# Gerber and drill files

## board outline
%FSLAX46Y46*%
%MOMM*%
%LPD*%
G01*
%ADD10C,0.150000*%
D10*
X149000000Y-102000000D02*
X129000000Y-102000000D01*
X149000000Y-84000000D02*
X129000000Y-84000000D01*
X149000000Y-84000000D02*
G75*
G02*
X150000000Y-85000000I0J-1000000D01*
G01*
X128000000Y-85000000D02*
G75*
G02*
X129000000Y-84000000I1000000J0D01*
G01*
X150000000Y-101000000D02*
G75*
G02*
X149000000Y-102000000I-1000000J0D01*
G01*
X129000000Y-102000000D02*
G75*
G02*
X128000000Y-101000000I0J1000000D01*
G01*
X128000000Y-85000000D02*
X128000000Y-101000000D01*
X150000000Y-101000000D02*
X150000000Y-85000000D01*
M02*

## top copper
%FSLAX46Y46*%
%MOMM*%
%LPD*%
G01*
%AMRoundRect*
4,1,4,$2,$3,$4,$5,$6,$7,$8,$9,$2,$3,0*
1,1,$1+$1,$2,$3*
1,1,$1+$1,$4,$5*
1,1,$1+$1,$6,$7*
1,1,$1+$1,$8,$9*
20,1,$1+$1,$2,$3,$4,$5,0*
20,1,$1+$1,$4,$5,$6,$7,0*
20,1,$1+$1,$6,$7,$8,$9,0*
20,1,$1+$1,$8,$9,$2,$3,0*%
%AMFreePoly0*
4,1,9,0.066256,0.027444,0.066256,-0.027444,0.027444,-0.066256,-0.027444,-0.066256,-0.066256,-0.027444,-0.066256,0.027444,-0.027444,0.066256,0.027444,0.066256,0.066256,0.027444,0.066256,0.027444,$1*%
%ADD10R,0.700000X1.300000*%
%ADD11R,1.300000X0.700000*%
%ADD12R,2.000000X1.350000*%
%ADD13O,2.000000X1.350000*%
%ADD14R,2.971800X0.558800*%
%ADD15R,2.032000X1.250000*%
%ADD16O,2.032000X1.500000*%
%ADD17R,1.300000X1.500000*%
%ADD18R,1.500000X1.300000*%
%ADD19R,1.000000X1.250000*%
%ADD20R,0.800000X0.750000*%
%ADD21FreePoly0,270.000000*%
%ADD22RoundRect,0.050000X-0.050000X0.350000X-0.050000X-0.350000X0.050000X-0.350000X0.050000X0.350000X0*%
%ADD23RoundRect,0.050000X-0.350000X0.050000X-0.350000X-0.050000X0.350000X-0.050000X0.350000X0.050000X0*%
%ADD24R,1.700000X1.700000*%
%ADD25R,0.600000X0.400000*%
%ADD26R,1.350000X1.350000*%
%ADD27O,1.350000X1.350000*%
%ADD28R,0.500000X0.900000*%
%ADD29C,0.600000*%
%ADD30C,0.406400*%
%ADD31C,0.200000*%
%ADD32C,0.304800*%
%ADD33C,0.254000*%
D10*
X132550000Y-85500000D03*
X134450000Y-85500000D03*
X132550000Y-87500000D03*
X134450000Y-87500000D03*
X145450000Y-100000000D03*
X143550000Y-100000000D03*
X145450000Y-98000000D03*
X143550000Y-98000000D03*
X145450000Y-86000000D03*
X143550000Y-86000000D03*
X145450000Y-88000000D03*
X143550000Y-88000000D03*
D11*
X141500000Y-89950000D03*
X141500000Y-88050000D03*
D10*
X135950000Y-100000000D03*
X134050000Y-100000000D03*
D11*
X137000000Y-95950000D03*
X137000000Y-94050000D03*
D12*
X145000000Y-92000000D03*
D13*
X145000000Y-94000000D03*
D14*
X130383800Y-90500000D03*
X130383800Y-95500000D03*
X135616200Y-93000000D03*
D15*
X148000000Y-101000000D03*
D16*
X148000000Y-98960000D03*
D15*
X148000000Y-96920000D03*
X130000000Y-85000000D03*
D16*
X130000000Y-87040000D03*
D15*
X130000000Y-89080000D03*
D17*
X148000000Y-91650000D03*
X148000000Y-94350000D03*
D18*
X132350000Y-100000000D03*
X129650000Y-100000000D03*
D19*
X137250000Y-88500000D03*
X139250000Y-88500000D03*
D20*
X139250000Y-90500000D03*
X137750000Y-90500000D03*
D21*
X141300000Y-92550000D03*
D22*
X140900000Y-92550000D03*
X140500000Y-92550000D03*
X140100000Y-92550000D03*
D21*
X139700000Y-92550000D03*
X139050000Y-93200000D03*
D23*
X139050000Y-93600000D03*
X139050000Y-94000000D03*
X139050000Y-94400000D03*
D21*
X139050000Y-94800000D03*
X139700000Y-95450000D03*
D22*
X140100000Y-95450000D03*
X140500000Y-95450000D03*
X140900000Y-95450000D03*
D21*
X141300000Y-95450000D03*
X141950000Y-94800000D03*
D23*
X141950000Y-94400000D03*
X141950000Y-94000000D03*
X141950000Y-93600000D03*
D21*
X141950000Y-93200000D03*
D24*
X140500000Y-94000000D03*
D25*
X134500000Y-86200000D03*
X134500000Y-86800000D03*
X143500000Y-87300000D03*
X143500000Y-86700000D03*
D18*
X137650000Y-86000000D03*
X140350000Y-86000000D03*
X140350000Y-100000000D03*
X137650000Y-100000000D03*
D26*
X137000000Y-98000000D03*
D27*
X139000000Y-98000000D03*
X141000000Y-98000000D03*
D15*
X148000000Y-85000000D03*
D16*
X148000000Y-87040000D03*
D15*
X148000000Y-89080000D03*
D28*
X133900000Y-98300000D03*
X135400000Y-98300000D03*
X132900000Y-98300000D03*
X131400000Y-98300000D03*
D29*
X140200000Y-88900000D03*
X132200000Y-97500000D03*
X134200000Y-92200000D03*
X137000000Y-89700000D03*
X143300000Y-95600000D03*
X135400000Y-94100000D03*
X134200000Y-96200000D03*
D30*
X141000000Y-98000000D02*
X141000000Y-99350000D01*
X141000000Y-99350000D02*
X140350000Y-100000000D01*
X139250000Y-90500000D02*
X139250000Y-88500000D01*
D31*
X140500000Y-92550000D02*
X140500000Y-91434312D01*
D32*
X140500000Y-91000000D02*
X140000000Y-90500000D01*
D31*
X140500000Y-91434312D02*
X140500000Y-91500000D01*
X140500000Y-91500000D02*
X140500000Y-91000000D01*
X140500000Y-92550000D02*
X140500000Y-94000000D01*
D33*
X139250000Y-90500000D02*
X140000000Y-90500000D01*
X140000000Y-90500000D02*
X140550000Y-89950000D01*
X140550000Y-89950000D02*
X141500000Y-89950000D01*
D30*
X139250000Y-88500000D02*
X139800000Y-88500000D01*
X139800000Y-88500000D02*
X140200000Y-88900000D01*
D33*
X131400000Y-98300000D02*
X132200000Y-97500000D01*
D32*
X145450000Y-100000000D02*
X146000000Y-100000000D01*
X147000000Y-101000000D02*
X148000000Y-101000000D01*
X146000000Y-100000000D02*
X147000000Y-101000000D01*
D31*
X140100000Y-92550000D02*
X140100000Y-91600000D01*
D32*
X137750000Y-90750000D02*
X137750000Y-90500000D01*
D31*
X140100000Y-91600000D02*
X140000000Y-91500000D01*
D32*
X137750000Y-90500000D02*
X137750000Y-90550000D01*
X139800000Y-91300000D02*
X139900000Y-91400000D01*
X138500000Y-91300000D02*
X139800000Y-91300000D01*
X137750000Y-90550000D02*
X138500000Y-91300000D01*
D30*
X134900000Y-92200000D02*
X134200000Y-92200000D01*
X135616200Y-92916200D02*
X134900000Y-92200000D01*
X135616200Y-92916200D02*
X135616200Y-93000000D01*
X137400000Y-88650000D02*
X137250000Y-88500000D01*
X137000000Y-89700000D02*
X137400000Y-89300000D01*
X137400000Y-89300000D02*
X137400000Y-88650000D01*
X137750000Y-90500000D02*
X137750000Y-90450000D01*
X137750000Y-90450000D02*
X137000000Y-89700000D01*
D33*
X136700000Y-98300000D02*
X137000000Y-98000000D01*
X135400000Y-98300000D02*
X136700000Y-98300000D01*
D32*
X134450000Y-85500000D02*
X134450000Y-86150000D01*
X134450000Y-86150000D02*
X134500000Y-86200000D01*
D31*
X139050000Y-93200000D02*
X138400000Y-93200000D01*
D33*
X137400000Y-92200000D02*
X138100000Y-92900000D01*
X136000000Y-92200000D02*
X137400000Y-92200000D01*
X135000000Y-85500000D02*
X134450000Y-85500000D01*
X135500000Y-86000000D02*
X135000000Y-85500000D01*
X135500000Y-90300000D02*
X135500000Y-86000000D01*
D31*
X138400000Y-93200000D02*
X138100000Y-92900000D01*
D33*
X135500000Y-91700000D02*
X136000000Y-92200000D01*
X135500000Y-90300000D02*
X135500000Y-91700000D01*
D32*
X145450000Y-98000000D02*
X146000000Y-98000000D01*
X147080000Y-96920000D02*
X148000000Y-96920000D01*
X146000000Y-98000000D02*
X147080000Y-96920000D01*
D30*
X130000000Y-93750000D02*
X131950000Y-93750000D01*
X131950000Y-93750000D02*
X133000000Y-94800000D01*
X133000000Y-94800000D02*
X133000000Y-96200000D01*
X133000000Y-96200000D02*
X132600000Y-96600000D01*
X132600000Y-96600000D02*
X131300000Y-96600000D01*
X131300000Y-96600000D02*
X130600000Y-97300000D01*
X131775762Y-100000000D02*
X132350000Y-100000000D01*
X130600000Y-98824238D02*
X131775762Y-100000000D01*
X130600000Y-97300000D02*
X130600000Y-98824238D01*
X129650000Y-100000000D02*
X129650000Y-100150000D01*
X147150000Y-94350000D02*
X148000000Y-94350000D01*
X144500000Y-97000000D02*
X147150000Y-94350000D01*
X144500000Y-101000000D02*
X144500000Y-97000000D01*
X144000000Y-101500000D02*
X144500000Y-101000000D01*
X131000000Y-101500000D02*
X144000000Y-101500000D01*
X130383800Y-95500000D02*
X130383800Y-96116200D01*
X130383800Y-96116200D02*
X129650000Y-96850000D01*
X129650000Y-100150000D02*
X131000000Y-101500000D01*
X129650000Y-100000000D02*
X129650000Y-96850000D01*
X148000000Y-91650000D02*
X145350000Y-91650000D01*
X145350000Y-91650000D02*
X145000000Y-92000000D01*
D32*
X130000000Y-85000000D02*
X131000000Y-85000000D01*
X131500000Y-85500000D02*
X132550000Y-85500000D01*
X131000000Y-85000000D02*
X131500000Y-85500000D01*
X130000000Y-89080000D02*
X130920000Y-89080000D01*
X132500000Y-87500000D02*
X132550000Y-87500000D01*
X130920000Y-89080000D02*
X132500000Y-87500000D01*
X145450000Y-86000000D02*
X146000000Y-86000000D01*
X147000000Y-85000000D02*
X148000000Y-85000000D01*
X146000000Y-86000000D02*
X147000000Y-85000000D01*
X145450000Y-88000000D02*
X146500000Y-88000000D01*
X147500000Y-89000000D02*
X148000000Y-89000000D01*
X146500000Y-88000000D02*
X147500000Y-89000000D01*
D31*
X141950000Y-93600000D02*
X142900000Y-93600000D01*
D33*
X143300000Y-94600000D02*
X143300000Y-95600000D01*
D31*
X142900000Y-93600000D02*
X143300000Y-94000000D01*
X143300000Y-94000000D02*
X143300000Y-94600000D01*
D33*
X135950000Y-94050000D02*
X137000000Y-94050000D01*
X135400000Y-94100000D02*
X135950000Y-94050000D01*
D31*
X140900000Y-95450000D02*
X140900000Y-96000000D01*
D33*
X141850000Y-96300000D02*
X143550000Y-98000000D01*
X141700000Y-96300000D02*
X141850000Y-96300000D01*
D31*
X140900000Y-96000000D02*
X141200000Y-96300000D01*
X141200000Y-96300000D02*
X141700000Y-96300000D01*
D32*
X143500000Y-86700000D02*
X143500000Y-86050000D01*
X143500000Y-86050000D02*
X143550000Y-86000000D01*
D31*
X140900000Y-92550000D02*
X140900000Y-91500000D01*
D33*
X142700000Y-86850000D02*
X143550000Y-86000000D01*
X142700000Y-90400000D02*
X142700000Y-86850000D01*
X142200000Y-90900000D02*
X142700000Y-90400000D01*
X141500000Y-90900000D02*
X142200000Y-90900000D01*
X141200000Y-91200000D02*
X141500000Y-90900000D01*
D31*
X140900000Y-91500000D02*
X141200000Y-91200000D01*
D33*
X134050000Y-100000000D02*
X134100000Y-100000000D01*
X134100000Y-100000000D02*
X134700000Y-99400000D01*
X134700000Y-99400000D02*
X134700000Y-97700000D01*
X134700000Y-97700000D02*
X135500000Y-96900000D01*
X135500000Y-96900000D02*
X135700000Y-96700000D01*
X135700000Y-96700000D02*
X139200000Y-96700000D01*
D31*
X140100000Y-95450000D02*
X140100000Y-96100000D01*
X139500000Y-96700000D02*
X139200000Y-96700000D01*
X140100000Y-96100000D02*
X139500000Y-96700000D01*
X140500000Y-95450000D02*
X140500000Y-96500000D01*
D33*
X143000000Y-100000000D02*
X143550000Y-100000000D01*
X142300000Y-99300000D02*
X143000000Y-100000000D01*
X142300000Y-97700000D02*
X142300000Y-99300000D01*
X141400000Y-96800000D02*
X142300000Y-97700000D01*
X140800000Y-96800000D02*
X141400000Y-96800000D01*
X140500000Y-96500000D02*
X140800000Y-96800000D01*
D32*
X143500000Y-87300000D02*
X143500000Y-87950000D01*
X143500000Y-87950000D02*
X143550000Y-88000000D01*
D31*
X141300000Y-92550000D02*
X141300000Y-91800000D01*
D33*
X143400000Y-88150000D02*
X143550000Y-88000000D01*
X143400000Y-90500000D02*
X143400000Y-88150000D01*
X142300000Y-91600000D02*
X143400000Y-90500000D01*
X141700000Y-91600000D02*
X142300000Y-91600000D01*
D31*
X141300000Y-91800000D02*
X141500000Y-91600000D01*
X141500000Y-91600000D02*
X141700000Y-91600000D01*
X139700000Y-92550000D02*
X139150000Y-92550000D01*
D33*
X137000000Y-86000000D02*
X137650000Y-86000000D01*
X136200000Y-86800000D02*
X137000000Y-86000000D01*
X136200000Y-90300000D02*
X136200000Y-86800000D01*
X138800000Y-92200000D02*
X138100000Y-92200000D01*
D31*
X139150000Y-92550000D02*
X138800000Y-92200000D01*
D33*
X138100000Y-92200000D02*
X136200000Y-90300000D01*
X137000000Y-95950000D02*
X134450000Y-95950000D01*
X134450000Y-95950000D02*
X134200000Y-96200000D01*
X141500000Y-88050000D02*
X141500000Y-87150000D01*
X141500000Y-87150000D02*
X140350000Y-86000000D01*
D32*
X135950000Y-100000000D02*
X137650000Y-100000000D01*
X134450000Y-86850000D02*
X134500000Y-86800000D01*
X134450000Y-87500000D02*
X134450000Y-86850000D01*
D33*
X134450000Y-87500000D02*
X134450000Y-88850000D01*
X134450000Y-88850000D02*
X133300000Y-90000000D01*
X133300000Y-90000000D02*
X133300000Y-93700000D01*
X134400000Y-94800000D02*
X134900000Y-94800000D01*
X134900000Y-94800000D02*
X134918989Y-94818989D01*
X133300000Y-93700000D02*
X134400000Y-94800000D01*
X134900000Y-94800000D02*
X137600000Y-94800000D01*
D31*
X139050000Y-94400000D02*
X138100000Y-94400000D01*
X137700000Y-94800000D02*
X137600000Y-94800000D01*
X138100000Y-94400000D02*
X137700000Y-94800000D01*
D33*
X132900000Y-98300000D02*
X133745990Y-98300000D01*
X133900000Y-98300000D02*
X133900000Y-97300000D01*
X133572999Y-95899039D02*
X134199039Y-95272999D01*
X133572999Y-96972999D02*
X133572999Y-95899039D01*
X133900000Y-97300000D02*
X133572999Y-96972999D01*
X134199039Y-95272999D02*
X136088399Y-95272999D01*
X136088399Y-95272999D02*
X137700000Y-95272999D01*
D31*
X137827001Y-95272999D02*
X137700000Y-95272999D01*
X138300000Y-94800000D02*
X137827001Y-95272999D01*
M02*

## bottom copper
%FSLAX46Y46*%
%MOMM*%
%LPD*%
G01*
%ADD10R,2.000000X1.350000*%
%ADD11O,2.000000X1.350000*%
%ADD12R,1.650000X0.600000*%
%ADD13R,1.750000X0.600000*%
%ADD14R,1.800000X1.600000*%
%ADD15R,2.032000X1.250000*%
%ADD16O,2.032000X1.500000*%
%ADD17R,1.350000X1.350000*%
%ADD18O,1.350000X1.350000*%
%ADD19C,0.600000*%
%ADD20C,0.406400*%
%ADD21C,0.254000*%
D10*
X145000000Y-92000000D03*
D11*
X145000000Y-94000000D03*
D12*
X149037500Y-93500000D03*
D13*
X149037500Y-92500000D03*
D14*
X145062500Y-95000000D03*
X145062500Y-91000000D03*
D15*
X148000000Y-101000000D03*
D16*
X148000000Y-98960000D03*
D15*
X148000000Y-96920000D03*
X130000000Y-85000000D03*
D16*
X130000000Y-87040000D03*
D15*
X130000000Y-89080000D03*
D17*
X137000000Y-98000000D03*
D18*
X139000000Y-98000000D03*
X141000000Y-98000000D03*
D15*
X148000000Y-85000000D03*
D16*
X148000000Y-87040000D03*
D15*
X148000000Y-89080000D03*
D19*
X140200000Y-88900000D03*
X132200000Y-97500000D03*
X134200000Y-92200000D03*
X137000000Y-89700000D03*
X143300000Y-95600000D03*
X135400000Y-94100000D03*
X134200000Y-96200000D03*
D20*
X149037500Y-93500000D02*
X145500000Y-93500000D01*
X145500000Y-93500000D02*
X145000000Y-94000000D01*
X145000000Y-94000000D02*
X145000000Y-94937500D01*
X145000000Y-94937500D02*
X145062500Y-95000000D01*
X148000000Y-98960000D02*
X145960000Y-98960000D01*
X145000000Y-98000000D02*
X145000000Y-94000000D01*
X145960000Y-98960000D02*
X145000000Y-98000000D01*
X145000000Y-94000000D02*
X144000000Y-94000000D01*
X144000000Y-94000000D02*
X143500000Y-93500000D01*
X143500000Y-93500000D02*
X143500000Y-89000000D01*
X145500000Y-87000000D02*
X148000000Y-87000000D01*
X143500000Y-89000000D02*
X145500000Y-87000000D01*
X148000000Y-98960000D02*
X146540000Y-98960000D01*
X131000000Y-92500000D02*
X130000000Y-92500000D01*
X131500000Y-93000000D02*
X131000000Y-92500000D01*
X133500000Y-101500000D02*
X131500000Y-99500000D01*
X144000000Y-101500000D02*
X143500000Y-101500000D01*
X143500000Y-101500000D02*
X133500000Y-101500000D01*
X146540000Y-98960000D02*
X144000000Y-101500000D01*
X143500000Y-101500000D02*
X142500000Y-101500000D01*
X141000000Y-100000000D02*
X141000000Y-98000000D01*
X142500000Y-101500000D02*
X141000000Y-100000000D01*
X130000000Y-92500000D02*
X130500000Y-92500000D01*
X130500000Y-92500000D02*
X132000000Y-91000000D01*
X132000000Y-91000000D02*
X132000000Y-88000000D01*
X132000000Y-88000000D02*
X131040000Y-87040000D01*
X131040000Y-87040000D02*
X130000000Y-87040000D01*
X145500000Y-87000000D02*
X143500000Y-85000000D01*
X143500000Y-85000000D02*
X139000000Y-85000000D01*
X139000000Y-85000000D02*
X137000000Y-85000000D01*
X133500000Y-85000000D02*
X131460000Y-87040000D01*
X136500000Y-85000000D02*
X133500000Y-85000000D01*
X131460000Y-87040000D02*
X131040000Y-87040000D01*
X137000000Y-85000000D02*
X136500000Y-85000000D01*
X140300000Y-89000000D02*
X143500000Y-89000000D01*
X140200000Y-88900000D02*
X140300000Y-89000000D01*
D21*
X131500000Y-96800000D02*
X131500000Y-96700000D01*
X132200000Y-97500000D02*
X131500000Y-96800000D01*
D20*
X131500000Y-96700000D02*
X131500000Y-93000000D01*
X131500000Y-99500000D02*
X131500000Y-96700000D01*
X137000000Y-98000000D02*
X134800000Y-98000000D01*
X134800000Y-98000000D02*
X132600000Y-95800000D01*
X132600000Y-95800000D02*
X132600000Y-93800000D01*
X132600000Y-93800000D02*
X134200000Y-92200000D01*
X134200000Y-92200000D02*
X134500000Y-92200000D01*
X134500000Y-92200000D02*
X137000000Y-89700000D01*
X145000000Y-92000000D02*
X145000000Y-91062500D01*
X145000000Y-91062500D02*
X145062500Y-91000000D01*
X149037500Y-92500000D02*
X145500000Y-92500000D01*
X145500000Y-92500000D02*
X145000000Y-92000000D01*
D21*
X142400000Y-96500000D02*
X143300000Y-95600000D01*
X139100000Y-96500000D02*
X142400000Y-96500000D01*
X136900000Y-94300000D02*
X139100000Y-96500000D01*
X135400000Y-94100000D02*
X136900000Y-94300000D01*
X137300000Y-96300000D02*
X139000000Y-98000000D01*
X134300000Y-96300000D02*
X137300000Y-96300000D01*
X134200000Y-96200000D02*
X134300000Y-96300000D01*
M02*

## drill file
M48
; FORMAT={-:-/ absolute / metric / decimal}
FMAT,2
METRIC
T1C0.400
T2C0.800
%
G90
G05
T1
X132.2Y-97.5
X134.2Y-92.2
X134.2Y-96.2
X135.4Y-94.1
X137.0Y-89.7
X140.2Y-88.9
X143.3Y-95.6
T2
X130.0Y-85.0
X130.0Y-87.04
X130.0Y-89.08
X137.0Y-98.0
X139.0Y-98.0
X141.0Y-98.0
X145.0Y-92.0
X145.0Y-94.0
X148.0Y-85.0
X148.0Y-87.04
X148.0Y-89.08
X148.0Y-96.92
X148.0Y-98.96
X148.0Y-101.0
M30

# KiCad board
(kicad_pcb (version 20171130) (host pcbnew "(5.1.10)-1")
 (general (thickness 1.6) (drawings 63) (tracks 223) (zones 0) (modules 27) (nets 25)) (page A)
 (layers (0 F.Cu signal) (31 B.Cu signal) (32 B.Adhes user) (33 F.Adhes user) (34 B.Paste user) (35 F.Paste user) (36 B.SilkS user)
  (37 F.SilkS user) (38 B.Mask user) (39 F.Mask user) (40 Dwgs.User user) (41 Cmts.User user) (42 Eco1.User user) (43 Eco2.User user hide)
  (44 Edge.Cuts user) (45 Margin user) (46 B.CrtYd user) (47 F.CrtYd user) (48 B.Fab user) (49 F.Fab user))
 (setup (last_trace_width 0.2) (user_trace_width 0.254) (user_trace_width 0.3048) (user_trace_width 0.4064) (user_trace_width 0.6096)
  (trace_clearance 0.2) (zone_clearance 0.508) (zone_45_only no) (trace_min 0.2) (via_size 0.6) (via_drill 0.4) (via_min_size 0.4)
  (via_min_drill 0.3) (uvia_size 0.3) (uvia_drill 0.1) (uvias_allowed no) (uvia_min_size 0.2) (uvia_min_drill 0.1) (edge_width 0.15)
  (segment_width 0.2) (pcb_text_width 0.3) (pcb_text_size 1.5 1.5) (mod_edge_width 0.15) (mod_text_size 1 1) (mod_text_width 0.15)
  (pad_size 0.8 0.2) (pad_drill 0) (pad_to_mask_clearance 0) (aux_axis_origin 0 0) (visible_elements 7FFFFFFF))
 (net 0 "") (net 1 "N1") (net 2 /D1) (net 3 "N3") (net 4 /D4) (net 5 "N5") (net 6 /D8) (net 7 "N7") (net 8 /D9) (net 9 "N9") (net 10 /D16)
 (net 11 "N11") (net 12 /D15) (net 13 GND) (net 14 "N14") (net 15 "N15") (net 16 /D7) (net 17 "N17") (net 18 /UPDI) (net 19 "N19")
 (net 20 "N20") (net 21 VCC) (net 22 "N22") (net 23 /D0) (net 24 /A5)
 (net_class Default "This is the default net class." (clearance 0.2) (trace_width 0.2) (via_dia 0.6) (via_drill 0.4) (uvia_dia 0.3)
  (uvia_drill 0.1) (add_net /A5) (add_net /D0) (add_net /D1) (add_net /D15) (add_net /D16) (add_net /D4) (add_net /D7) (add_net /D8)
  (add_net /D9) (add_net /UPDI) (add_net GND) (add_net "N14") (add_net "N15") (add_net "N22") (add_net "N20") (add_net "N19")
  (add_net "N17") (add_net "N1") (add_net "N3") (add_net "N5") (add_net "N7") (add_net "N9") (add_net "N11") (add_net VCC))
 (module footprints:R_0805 (layer F.Cu) (at 133.5 85.5 180)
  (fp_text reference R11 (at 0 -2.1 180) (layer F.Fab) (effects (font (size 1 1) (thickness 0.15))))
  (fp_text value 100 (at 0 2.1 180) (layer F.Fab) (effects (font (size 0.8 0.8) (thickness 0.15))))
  (pad 2 smd rect (at 0.95 0 180) (size 0.7 1.3) (layers F.Cu F.Paste F.Mask) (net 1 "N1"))
  (pad 1 smd rect (at -0.95 0 180) (size 0.7 1.3) (layers F.Cu F.Paste F.Mask) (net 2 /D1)))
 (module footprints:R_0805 (layer F.Cu) (at 133.5 87.5 180)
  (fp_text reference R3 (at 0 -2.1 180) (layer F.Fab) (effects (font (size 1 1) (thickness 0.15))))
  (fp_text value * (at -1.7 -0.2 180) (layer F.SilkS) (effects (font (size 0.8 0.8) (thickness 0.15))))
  (pad 2 smd rect (at 0.95 0 180) (size 0.7 1.3) (layers F.Cu F.Paste F.Mask) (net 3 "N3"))
  (pad 1 smd rect (at -0.95 0 180) (size 0.7 1.3) (layers F.Cu F.Paste F.Mask) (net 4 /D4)))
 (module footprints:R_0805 (layer F.Cu) (at 144.5 100)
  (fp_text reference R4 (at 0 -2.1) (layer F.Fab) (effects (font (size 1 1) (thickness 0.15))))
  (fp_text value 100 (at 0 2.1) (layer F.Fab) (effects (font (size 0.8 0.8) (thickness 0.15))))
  (pad 2 smd rect (at 0.95 0) (size 0.7 1.3) (layers F.Cu F.Paste F.Mask) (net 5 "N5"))
  (pad 1 smd rect (at -0.95 0) (size 0.7 1.3) (layers F.Cu F.Paste F.Mask) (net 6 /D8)))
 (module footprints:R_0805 (layer F.Cu) (at 144.5 98)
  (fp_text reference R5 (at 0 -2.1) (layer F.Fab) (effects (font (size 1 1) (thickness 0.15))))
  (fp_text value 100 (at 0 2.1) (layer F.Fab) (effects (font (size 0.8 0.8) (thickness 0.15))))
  (pad 2 smd rect (at 0.95 0) (size 0.7 1.3) (layers F.Cu F.Paste F.Mask) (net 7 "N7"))
  (pad 1 smd rect (at -0.95 0) (size 0.7 1.3) (layers F.Cu F.Paste F.Mask) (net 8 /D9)))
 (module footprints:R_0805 (layer F.Cu) (at 144.5 86)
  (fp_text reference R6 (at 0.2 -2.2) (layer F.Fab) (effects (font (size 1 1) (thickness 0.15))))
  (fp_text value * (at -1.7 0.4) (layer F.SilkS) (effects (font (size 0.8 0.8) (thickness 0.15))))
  (pad 2 smd rect (at 0.95 0) (size 0.7 1.3) (layers F.Cu F.Paste F.Mask) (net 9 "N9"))
  (pad 1 smd rect (at -0.95 0) (size 0.7 1.3) (layers F.Cu F.Paste F.Mask) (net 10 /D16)))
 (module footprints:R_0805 (layer F.Cu) (at 144.5 88)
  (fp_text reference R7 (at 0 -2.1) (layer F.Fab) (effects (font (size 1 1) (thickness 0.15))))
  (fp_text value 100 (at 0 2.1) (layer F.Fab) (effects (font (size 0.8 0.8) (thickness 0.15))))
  (pad 2 smd rect (at 0.95 0) (size 0.7 1.3) (layers F.Cu F.Paste F.Mask) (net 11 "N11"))
  (pad 1 smd rect (at -0.95 0) (size 0.7 1.3) (layers F.Cu F.Paste F.Mask) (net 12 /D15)))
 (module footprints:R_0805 (layer F.Cu) (at 141.5 89 270)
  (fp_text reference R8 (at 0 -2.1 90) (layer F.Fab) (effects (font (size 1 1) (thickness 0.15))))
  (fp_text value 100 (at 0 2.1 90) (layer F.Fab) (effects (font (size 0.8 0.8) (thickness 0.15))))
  (pad 2 smd rect (at 0.95 0 270) (size 0.7 1.3) (layers F.Cu F.Paste F.Mask) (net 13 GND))
  (pad 1 smd rect (at -0.95 0 270) (size 0.7 1.3) (layers F.Cu F.Paste F.Mask) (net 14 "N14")))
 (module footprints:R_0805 (layer F.Cu) (at 135 100)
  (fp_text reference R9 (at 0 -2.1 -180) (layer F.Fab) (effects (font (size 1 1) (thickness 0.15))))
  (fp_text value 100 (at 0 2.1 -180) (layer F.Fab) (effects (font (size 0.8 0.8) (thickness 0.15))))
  (pad 2 smd rect (at 0.95 0) (size 0.7 1.3) (layers F.Cu F.Paste F.Mask) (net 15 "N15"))
  (pad 1 smd rect (at -0.95 0) (size 0.7 1.3) (layers F.Cu F.Paste F.Mask) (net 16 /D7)))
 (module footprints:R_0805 (layer F.Cu) (at 137 95 270)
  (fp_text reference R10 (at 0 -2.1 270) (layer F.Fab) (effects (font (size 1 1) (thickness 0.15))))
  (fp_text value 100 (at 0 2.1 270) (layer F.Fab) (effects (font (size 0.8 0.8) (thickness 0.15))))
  (pad 2 smd rect (at 0.95 0 270) (size 0.7 1.3) (layers F.Cu F.Paste F.Mask) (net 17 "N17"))
  (pad 1 smd rect (at -0.95 0 270) (size 0.7 1.3) (layers F.Cu F.Paste F.Mask) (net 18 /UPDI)))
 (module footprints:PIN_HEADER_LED (layer B.Cu) (at 145 92 180)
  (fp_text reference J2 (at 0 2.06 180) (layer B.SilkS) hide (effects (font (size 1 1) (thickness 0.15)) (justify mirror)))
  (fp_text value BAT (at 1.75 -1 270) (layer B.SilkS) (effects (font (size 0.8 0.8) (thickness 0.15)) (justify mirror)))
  (pad 1 thru_hole rect (at 0 0 180) (size 2 1.35) (drill 0.8) (layers *.Cu *.Mask) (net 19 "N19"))
  (pad 2 thru_hole oval (at 0 -2 180) (size 2 1.35) (drill 0.8) (layers *.Cu *.Mask) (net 13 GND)))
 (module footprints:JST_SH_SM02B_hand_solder (layer B.Cu) (at 147 93 90)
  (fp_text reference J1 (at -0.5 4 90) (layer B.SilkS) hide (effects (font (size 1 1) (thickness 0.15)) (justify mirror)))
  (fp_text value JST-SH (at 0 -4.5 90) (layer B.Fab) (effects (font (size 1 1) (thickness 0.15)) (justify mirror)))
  (pad 1 smd rect (at -0.5 2.0375 90) (size 0.6 1.65) (layers B.Cu B.Paste B.Mask) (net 13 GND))
  (pad 2 smd rect (at 0.5 2.0375 90) (size 0.6 1.75) (layers B.Cu B.Paste B.Mask) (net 19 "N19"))
  (pad 1 smd rect (at -2 -1.9375 90) (size 1.6 1.8) (layers B.Cu B.Paste B.Mask) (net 13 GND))
  (pad 2 smd rect (at 2 -1.9375 90) (size 1.6 1.8) (layers B.Cu B.Paste B.Mask) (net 19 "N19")))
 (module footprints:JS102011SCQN (layer F.Cu) (at 133 93)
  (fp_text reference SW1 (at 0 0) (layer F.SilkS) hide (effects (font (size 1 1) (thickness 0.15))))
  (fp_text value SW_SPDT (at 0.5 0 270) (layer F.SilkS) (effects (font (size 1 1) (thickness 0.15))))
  (pad 1 smd rect (at -2.6162 -2.5) (size 2.9718 0.5588) (layers F.Cu F.Paste F.Mask))
  (pad 3 smd rect (at -2.6162 2.5) (size 2.9718 0.5588) (layers F.Cu F.Paste F.Mask) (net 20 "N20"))
  (pad 2 smd rect (at 2.6162 0) (size 2.9718 0.5588) (layers F.Cu F.Paste F.Mask) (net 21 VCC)))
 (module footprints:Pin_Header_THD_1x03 (layer F.Cu) (at 148 101 180)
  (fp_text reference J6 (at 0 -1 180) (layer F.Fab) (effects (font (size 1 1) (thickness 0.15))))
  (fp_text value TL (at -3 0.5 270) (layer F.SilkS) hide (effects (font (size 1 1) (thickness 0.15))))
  (pad 1 thru_hole rect (at 0 0 180) (size 2.032 1.25) (drill 0.8) (layers *.Cu *.Mask F.SilkS) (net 5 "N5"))
  (pad 2 thru_hole oval (at 0 2.04 180) (size 2.032 1.5) (drill 0.8) (layers *.Cu *.Mask F.SilkS) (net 13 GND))
  (pad 3 thru_hole rect (at 0 4.08 180) (size 2.032 1.25) (drill 0.8) (layers *.Cu *.Mask F.SilkS) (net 7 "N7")))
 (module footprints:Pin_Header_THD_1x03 (layer F.Cu) (at 130 85)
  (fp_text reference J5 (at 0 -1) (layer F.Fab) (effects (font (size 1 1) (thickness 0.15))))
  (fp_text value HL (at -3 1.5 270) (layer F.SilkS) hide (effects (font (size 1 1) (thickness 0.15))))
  (pad 1 thru_hole rect (at 0 0) (size 2.032 1.25) (drill 0.8) (layers *.Cu *.Mask F.SilkS) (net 1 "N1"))
  (pad 2 thru_hole oval (at 0 2.04) (size 2.032 1.5) (drill 0.8) (layers *.Cu *.Mask F.SilkS) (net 13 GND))
  (pad 3 thru_hole rect (at 0 4.08) (size 2.032 1.25) (drill 0.8) (layers *.Cu *.Mask F.SilkS) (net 3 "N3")))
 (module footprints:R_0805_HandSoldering (layer F.Cu) (at 148 93 270)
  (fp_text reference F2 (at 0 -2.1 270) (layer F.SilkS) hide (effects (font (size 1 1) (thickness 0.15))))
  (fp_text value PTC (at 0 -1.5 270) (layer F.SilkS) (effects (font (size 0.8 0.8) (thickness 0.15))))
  (pad 1 smd rect (at -1.35 0 270) (size 1.5 1.3) (layers F.Cu F.Paste F.Mask) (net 19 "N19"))
  (pad 2 smd rect (at 1.35 0 270) (size 1.5 1.3) (layers F.Cu F.Paste F.Mask) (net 20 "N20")))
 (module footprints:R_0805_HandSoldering (layer F.Cu) (at 131 100 180)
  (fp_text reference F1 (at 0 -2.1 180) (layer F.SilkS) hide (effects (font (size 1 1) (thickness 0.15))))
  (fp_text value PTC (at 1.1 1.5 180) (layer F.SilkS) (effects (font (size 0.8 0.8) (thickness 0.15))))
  (pad 1 smd rect (at -1.35 0 180) (size 1.5 1.3) (layers F.Cu F.Paste F.Mask) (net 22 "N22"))
  (pad 2 smd rect (at 1.35 0 180) (size 1.5 1.3) (layers F.Cu F.Paste F.Mask) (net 20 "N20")))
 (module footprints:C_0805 (layer F.Cu) (at 138.25 88.5)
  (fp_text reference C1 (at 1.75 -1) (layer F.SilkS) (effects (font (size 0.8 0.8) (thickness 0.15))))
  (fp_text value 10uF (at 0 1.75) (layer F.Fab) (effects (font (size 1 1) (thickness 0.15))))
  (pad 1 smd rect (at -1 0) (size 1 1.25) (layers F.Cu F.Paste F.Mask) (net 21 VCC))
  (pad 2 smd rect (at 1 0) (size 1 1.25) (layers F.Cu F.Paste F.Mask) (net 13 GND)))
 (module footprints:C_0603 (layer F.Cu) (at 138.5 90.5)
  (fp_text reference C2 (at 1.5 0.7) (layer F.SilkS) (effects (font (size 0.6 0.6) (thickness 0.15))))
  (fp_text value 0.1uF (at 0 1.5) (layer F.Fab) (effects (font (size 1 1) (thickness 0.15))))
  (pad 2 smd rect (at 0.75 0) (size 0.8 0.75) (layers F.Cu F.Paste F.Mask) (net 13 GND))
  (pad 1 smd rect (at -0.75 0) (size 0.8 0.75) (layers F.Cu F.Paste F.Mask) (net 21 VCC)))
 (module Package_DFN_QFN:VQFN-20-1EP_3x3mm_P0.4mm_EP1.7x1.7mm (layer F.Cu) (at 140.5 94 270)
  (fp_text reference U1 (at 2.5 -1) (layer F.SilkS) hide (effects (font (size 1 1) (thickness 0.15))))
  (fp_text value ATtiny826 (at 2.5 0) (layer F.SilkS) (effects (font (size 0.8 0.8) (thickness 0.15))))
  (pad 1 smd custom (at -1.45 -0.8 270) (size 0.143431 0.143431) (layers F.Cu F.Paste F.Mask) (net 12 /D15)
   (options (clearance outline) (anchor circle)) (primitives))
  (pad 2 smd roundrect (at -1.45 -0.4 270) (size 0.8 0.2) (layers F.Cu F.Paste F.Mask) (roundrect_rratio 0.25) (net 10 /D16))
  (pad 3 smd roundrect (at -1.45 0 270) (size 0.8 0.2) (layers F.Cu F.Paste F.Mask) (roundrect_rratio 0.25) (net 13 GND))
  (pad 4 smd roundrect (at -1.45 0.4 270) (size 0.8 0.2) (layers F.Cu F.Paste F.Mask) (roundrect_rratio 0.25) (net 21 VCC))
  (pad 5 smd custom (at -1.45 0.8 270) (size 0.143431 0.143431) (layers F.Cu F.Paste F.Mask) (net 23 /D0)
   (options (clearance outline) (anchor circle)) (primitives))
  (pad 6 smd custom (at -0.8 1.45 270) (size 0.143431 0.143431) (layers F.Cu F.Paste F.Mask) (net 2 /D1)
   (options (clearance outline) (anchor circle)) (primitives))
  (pad 7 smd roundrect (at -0.4 1.45 270) (size 0.2 0.8) (layers F.Cu F.Paste F.Mask) (roundrect_rratio 0.25))
  (pad 8 smd roundrect (at 0 1.45 270) (size 0.2 0.8) (layers F.Cu F.Paste F.Mask) (roundrect_rratio 0.25))
  (pad 9 smd roundrect (at 0.4 1.45 270) (size 0.2 0.8) (layers F.Cu F.Paste F.Mask) (roundrect_rratio 0.25) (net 4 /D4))
  (pad 10 smd custom (at 0.8 1.45 270) (size 0.143431 0.143431) (layers F.Cu F.Paste F.Mask) (options (clearance outline) (anchor circle))
   (primitives))
  (pad 11 smd custom (at 1.45 0.8 270) (size 0.143431 0.143431) (layers F.Cu F.Paste F.Mask) (options (clearance outline) (anchor circle))
   (primitives))
  (pad 12 smd roundrect (at 1.45 0.4 270) (size 0.8 0.2) (layers F.Cu F.Paste F.Mask) (roundrect_rratio 0.25) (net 16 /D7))
  (pad 13 smd roundrect (at 1.45 0 270) (size 0.8 0.2) (layers F.Cu F.Paste F.Mask) (roundrect_rratio 0.25) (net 6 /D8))
  (pad 14 smd roundrect (at 1.45 -0.4 270) (size 0.8 0.2) (layers F.Cu F.Paste F.Mask) (roundrect_rratio 0.25) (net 8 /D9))
  (pad 15 smd custom (at 1.45 -0.8 270) (size 0.143431 0.143431) (layers F.Cu F.Paste F.Mask) (options (clearance outline) (anchor circle))
   (primitives))
  (pad 16 smd custom (at 0.8 -1.45 270) (size 0.143431 0.143431) (layers F.Cu F.Paste F.Mask) (options (clearance outline) (anchor circle))
   (primitives))
  (pad 17 smd roundrect (at 0.4 -1.45 270) (size 0.2 0.8) (layers F.Cu F.Paste F.Mask) (roundrect_rratio 0.25))
  (pad 18 smd roundrect (at 0 -1.45 270) (size 0.2 0.8) (layers F.Cu F.Paste F.Mask) (roundrect_rratio 0.25))
  (pad 19 smd roundrect (at -0.4 -1.45 270) (size 0.2 0.8) (layers F.Cu F.Paste F.Mask) (roundrect_rratio 0.25) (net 18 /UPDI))
  (pad 20 smd custom (at -0.8 -1.45 270) (size 0.143431 0.143431) (layers F.Cu F.Paste F.Mask) (options (clearance outline) (anchor circle))
   (primitives))
  (pad 21 smd rect (at 0 0 270) (size 1.7 1.7) (layers F.Cu F.Mask) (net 13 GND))
  (pad "" smd roundrect (at -0.425 -0.425 270) (size 0.69 0.69) (layers F.Paste) (roundrect_rratio 0.25))
  (pad "" smd roundrect (at -0.425 0.425 270) (size 0.69 0.69) (layers F.Paste) (roundrect_rratio 0.25))
  (pad "" smd roundrect (at 0.425 -0.425 270) (size 0.69 0.69) (layers F.Paste) (roundrect_rratio 0.25))
  (pad "" smd roundrect (at 0.425 0.425 270) (size 0.69 0.69) (layers F.Paste) (roundrect_rratio 0.25)))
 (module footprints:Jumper (layer F.Cu) (at 134.5 86.5 270)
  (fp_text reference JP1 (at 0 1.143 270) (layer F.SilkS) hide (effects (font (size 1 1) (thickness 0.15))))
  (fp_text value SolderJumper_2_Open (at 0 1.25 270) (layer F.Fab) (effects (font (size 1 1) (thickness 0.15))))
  (pad 1 smd rect (at -0.3 0 270) (size 0.4 0.6) (layers F.Cu F.Paste F.Mask) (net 2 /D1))
  (pad 2 smd rect (at 0.3 0 270) (size 0.4 0.6) (layers F.Cu F.Paste F.Mask) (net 4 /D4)))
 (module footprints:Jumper (layer F.Cu) (at 143.5 87 270)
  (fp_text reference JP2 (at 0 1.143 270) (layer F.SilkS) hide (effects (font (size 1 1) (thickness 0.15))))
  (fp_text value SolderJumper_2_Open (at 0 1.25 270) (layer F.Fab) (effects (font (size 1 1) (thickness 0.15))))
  (pad 2 smd rect (at 0.3 0 270) (size 0.4 0.6) (layers F.Cu F.Paste F.Mask) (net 12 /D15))
  (pad 1 smd rect (at -0.3 0 270) (size 0.4 0.6) (layers F.Cu F.Paste F.Mask) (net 10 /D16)))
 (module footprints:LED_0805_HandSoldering (layer F.Cu) (at 139 86 180)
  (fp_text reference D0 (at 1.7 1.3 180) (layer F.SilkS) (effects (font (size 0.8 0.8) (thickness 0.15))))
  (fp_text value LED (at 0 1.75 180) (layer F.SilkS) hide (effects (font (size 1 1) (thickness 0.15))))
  (pad 2 smd rect (at 1.35 0 180) (size 1.5 1.3) (layers F.Cu F.Paste F.Mask) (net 23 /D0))
  (pad 1 smd rect (at -1.35 0 180) (size 1.5 1.3) (layers F.Cu F.Paste F.Mask) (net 14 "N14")))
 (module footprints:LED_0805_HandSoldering (layer F.Cu) (at 139 100 180)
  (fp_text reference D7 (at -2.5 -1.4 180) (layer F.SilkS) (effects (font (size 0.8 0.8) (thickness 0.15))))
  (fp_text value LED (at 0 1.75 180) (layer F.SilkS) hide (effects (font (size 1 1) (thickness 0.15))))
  (pad 1 smd rect (at -1.35 0 180) (size 1.5 1.3) (layers F.Cu F.Paste F.Mask) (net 13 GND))
  (pad 2 smd rect (at 1.35 0 180) (size 1.5 1.3) (layers F.Cu F.Paste F.Mask) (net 15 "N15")))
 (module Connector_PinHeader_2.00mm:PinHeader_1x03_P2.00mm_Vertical (layer B.Cu) (at 137 98 270)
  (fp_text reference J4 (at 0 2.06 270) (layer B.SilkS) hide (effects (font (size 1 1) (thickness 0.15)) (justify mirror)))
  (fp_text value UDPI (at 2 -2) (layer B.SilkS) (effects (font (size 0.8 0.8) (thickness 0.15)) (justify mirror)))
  (pad 1 thru_hole rect (at 0 0 270) (size 1.35 1.35) (drill 0.8) (layers *.Cu *.Mask) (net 21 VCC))
  (pad 2 thru_hole oval (at 0 -2 270) (size 1.35 1.35) (drill 0.8) (layers *.Cu *.Mask) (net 17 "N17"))
  (pad 3 thru_hole oval (at 0 -4 270) (size 1.35 1.35) (drill 0.8) (layers *.Cu *.Mask) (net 13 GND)))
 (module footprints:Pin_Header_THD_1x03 (layer F.Cu) (at 148 85)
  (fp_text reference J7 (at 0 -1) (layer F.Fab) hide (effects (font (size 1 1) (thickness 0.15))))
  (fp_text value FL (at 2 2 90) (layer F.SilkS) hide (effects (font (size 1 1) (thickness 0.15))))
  (pad 1 thru_hole rect (at 0 0) (size 2.032 1.25) (drill 0.8) (layers *.Cu *.Mask F.SilkS) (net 9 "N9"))
  (pad 2 thru_hole oval (at 0 2.04) (size 2.032 1.5) (drill 0.8) (layers *.Cu *.Mask F.SilkS) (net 13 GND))
  (pad 3 thru_hole rect (at 0 4.08) (size 2.032 1.25) (drill 0.8) (layers *.Cu *.Mask F.SilkS) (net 11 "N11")))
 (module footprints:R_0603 (layer F.Cu) (at 134.65 98.3 180)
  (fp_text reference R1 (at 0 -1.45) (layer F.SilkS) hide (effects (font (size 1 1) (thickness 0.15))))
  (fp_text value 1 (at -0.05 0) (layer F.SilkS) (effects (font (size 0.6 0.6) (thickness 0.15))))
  (pad 2 smd rect (at 0.75 0 180) (size 0.5 0.9) (layers F.Cu F.Paste F.Mask) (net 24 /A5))
  (pad 1 smd rect (at -0.75 0 180) (size 0.5 0.9) (layers F.Cu F.Paste F.Mask) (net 21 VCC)))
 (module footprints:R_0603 (layer F.Cu) (at 132.15 98.3 180)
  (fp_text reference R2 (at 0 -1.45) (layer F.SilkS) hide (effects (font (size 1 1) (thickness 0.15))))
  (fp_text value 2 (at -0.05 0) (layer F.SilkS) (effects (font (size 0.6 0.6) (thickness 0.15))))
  (pad 1 smd rect (at -0.75 0 180) (size 0.5 0.9) (layers F.Cu F.Paste F.Mask) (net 24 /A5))
  (pad 2 smd rect (at 0.75 0 180) (size 0.5 0.9) (layers F.Cu F.Paste F.Mask) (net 13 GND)))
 (gr_line (start 149 102) (end 129 102) (angle 90) (layer Edge.Cuts) (width 0.15))
 (gr_line (start 149 84) (end 129 84) (angle 90) (layer Edge.Cuts) (width 0.15))
 (gr_arc (start 149 85) (end 149 84) (angle 90) (layer Edge.Cuts) (width 0.15))
 (gr_arc (start 129 85) (end 128 85) (angle 90) (layer Edge.Cuts) (width 0.15))
 (gr_arc (start 149 101) (end 150 101) (angle 90) (layer Edge.Cuts) (width 0.15))
 (gr_arc (start 129 101) (end 129 102) (angle 90) (layer Edge.Cuts) (width 0.15))
 (gr_line (start 128 85) (end 128 101) (angle 90) (layer Edge.Cuts) (width 0.15))
 (gr_line (start 150 101) (end 150 85) (angle 90) (layer Edge.Cuts) (width 0.15))
 (segment (start 149.0375 93.5) (end 145.5 93.5) (width 0.4064) (layer B.Cu) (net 13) (status C00030))
 (segment (start 145.5 93.5) (end 145 94) (width 0.4064) (layer B.Cu) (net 13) (status C00030))
 (segment (start 145 94) (end 145 94.9375) (width 0.4064) (layer B.Cu) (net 13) (status C00030))
 (segment (start 145 94.9375) (end 145.0625 95) (width 0.4064) (layer B.Cu) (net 13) (status C00030))
 (segment (start 148 98.96) (end 145.96 98.96) (width 0.4064) (layer B.Cu) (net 13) (status 400010))
 (segment (start 145 98) (end 145 94) (width 0.4064) (layer B.Cu) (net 13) (status 800020))
 (segment (start 145.96 98.96) (end 145 98) (width 0.4064) (layer B.Cu) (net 13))
 (segment (start 145 94) (end 144 94) (width 0.4064) (layer B.Cu) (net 13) (status C00030))
 (segment (start 144 94) (end 143.5 93.5) (width 0.4064) (layer B.Cu) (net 13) (status 400010))
 (segment (start 143.5 93.5) (end 143.5 89) (width 0.4064) (layer B.Cu) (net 13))
 (segment (start 145.5 87) (end 148 87) (width 0.4064) (layer B.Cu) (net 13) (status 800020))
 (segment (start 143.5 89) (end 145.5 87) (width 0.4064) (layer B.Cu) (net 13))
 (segment (start 148 98.96) (end 146.54 98.96) (width 0.4064) (layer B.Cu) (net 13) (status 400010))
 (segment (start 131 92.5) (end 130 92.5) (width 0.4064) (layer B.Cu) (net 13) (status 800020))
 (segment (start 131.5 93) (end 131 92.5) (width 0.4064) (layer B.Cu) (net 13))
 (segment (start 133.5 101.5) (end 131.5 99.5) (width 0.4064) (layer B.Cu) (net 13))
 (segment (start 144 101.5) (end 143.5 101.5) (width 0.4064) (layer B.Cu) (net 13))
 (segment (start 143.5 101.5) (end 133.5 101.5) (width 0.4064) (layer B.Cu) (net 13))
 (segment (start 146.54 98.96) (end 144 101.5) (width 0.4064) (layer B.Cu) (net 13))
 (segment (start 143.5 101.5) (end 142.5 101.5) (width 0.4064) (layer B.Cu) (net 13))
 (segment (start 141 100) (end 141 98) (width 0.4064) (layer B.Cu) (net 13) (status 800020))
 (segment (start 142.5 101.5) (end 141 100) (width 0.4064) (layer B.Cu) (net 13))
 (segment (start 141 98) (end 141 99.35) (width 0.4064) (layer F.Cu) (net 13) (status C00030))
 (segment (start 141 99.35) (end 140.35 100) (width 0.4064) (layer F.Cu) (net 13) (status C00030))
 (segment (start 130 92.5) (end 130.5 92.5) (width 0.4064) (layer B.Cu) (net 13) (status C00030))
 (segment (start 130.5 92.5) (end 132 91) (width 0.4064) (layer B.Cu) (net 13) (status 400010))
 (segment (start 132 91) (end 132 88) (width 0.4064) (layer B.Cu) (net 13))
 (segment (start 132 88) (end 131.04 87.04) (width 0.4064) (layer B.Cu) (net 13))
 (segment (start 131.04 87.04) (end 130 87.04) (width 0.4064) (layer B.Cu) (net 13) (status 800020))
 (segment (start 145.5 87) (end 143.5 85) (width 0.4064) (layer B.Cu) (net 13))
 (segment (start 143.5 85) (end 139 85) (width 0.4064) (layer B.Cu) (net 13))
 (segment (start 139 85) (end 137 85) (width 0.4064) (layer B.Cu) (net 13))
 (segment (start 133.5 85) (end 131.46 87.04) (width 0.4064) (layer B.Cu) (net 13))
 (segment (start 136.5 85) (end 133.5 85) (width 0.4064) (layer B.Cu) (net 13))
 (segment (start 131.46 87.04) (end 131.04 87.04) (width 0.4064) (layer B.Cu) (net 13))
 (segment (start 137 85) (end 136.5 85) (width 0.4064) (layer B.Cu) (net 13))
 (segment (start 139.25 90.5) (end 139.25 88.5) (width 0.4064) (layer F.Cu) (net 13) (status C00030))
 (segment (start 140.5 92.55) (end 140.5 91.434312) (width 0.2) (layer F.Cu) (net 13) (status 400010))
 (segment (start 140.5 91) (end 140 90.5) (width 0.3048) (layer F.Cu) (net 13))
 (segment (start 140.5 91.434312) (end 140.5 91.5) (width 0.2) (layer F.Cu) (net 13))
 (segment (start 140.5 91.5) (end 140.5 91) (width 0.2) (layer F.Cu) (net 13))
 (segment (start 140.5 92.55) (end 140.5 94) (width 0.2) (layer F.Cu) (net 13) (status C00030))
 (segment (start 139.25 90.5) (end 140 90.5) (width 0.254) (layer F.Cu) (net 13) (status 400010))
 (segment (start 140 90.5) (end 140.55 89.95) (width 0.254) (layer F.Cu) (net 13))
 (segment (start 140.55 89.95) (end 141.5 89.95) (width 0.254) (layer F.Cu) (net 13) (status 800020))
 (segment (start 139.25 88.5) (end 139.8 88.5) (width 0.4064) (layer F.Cu) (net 13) (status 400010))
 (segment (start 140.3 89) (end 143.5 89) (width 0.4064) (layer B.Cu) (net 13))
 (segment (start 140.2 88.9) (end 140.3 89) (width 0.4064) (layer B.Cu) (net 13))
 (via (at 140.2 88.9) (size 0.6) (drill 0.4) (layers F.Cu B.Cu) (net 13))
 (segment (start 139.8 88.5) (end 140.2 88.9) (width 0.4064) (layer F.Cu) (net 13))
 (via (at 132.2 97.5) (size 0.6) (drill 0.4) (layers F.Cu B.Cu) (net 13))
 (segment (start 131.4 98.3) (end 132.2 97.5) (width 0.254) (layer F.Cu) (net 13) (status 10))
 (segment (start 131.5 96.8) (end 131.5 96.7) (width 0.254) (layer B.Cu) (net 13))
 (segment (start 132.2 97.5) (end 131.5 96.8) (width 0.254) (layer B.Cu) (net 13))
 (segment (start 131.5 96.7) (end 131.5 93) (width 0.4064) (layer B.Cu) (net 13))
 (segment (start 131.5 99.5) (end 131.5 96.7) (width 0.4064) (layer B.Cu) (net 13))
 (segment (start 145.45 100) (end 146 100) (width 0.3048) (layer F.Cu) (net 5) (status 400010))
 (segment (start 147 101) (end 148 101) (width 0.3048) (layer F.Cu) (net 5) (status C00030))
 (segment (start 146 100) (end 147 101) (width 0.3048) (layer F.Cu) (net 5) (status 800020))
 (segment (start 140.1 92.55) (end 140.1 91.6) (width 0.2) (layer F.Cu) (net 21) (status 400010))
 (segment (start 137.75 90.75) (end 137.75 90.5) (width 0.3048) (layer F.Cu) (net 21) (status C00030))
 (segment (start 140.1 91.6) (end 140 91.5) (width 0.2) (layer F.Cu) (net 21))
 (segment (start 137.75 90.5) (end 137.75 90.55) (width 0.3048) (layer F.Cu) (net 21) (status C00030))
 (segment (start 139.8 91.3) (end 139.9 91.4) (width 0.3048) (layer F.Cu) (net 21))
 (segment (start 138.5 91.3) (end 139.8 91.3) (width 0.3048) (layer F.Cu) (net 21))
 (segment (start 137.75 90.55) (end 138.5 91.3) (width 0.3048) (layer F.Cu) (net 21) (status 400010))
 (segment (start 137 98) (end 134.8 98) (width 0.4064) (layer B.Cu) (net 21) (status 400010))
 (segment (start 134.9 92.2) (end 134.2 92.2) (width 0.4064) (layer F.Cu) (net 21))
 (segment (start 135.6162 92.9162) (end 134.9 92.2) (width 0.4064) (layer F.Cu) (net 21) (status 400010))
 (segment (start 135.6162 92.9162) (end 135.6162 93) (width 0.4064) (layer F.Cu) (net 21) (status C00030))
 (segment (start 134.8 98) (end 132.6 95.8) (width 0.4064) (layer B.Cu) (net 21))
 (segment (start 132.6 95.8) (end 132.6 93.8) (width 0.4064) (layer B.Cu) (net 21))
 (segment (start 132.6 93.8) (end 134.2 92.2) (width 0.4064) (layer B.Cu) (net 21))
 (via (at 134.2 92.2) (size 0.6) (drill 0.4) (layers F.Cu B.Cu) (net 21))
 (segment (start 134.2 92.2) (end 134.5 92.2) (width 0.4064) (layer B.Cu) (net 21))
 (via (at 137 89.7) (size 0.6) (drill 0.4) (layers F.Cu B.Cu) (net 21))
 (segment (start 134.5 92.2) (end 137 89.7) (width 0.4064) (layer B.Cu) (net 21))
 (segment (start 137.4 88.65) (end 137.25 88.5) (width 0.4064) (layer F.Cu) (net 21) (status C00030))
 (segment (start 137 89.7) (end 137.4 89.3) (width 0.4064) (layer F.Cu) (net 21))
 (segment (start 137.4 89.3) (end 137.4 88.65) (width 0.4064) (layer F.Cu) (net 21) (status 800020))
 (segment (start 137.75 90.5) (end 137.75 90.45) (width 0.4064) (layer F.Cu) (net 21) (status C00030))
 (segment (start 137.75 90.45) (end 137 89.7) (width 0.4064) (layer F.Cu) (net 21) (status 400010))
 (segment (start 136.7 98.3) (end 137 98) (width 0.254) (layer F.Cu) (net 21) (status 30))
 (segment (start 135.4 98.3) (end 136.7 98.3) (width 0.254) (layer F.Cu) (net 21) (status 30))
 (segment (start 134.45 85.5) (end 134.45 86.15) (width 0.3048) (layer F.Cu) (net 2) (status C00030))
 (segment (start 134.45 86.15) (end 134.5 86.2) (width 0.3048) (layer F.Cu) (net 2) (status C00030))
 (segment (start 139.05 93.2) (end 138.4 93.2) (width 0.2) (layer F.Cu) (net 2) (status 400010))
 (segment (start 137.4 92.2) (end 138.1 92.9) (width 0.254) (layer F.Cu) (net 2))
 (segment (start 136 92.2) (end 137.4 92.2) (width 0.254) (layer F.Cu) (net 2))
 (segment (start 135 85.5) (end 134.45 85.5) (width 0.254) (layer F.Cu) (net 2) (status 800020))
 (segment (start 135.5 86) (end 135 85.5) (width 0.254) (layer F.Cu) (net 2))
 (segment (start 135.5 90.3) (end 135.5 86) (width 0.254) (layer F.Cu) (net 2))
 (segment (start 138.4 93.2) (end 138.1 92.9) (width 0.2) (layer F.Cu) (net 2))
 (segment (start 135.5 91.7) (end 136 92.2) (width 0.254) (layer F.Cu) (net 2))
 (segment (start 135.5 90.3) (end 135.5 91.7) (width 0.254) (layer F.Cu) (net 2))
 (segment (start 145.45 98) (end 146 98) (width 0.3048) (layer F.Cu) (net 7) (status 400010))
 (segment (start 147.08 96.92) (end 148 96.92) (width 0.3048) (layer F.Cu) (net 7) (status C00030))
 (segment (start 146 98) (end 147.08 96.92) (width 0.3048) (layer F.Cu) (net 7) (status 800020))
 (segment (start 130 93.75) (end 131.95 93.75) (width 0.4064) (layer F.Cu) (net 22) (status 10))
 (segment (start 131.95 93.75) (end 133 94.8) (width 0.4064) (layer F.Cu) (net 22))
 (segment (start 133 94.8) (end 133 96.2) (width 0.4064) (layer F.Cu) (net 22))
 (segment (start 133 96.2) (end 132.6 96.6) (width 0.4064) (layer F.Cu) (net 22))
 (segment (start 132.6 96.6) (end 131.3 96.6) (width 0.4064) (layer F.Cu) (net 22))
 (segment (start 131.3 96.6) (end 130.6 97.3) (width 0.4064) (layer F.Cu) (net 22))
 (segment (start 131.775762 100) (end 132.35 100) (width 0.4064) (layer F.Cu) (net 22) (status 30))
 (segment (start 130.6 98.824238) (end 131.775762 100) (width 0.4064) (layer F.Cu) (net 22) (status 20))
 (segment (start 130.6 97.3) (end 130.6 98.824238) (width 0.4064) (layer F.Cu) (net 22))
 (segment (start 129.65 100) (end 129.65 100.15) (width 0.4064) (layer F.Cu) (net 20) (status C00030))
 (segment (start 147.15 94.35) (end 148 94.35) (width 0.4064) (layer F.Cu) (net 20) (status 800020))
 (segment (start 144.5 97) (end 147.15 94.35) (width 0.4064) (layer F.Cu) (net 20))
 (segment (start 144.5 101) (end 144.5 97) (width 0.4064) (layer F.Cu) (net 20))
 (segment (start 144 101.5) (end 144.5 101) (width 0.4064) (layer F.Cu) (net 20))
 (segment (start 131 101.5) (end 144 101.5) (width 0.4064) (layer F.Cu) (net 20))
 (segment (start 130.3838 95.5) (end 130.3838 96.1162) (width 0.4064) (layer F.Cu) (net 20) (status 400010))
 (segment (start 130.3838 96.1162) (end 129.65 96.85) (width 0.4064) (layer F.Cu) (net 20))
 (segment (start 129.65 100.15) (end 131 101.5) (width 0.4064) (layer F.Cu) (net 20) (status 400010))
 (segment (start 129.65 100) (end 129.65 96.85) (width 0.4064) (layer F.Cu) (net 20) (status 10))
 (segment (start 148 91.65) (end 145.35 91.65) (width 0.4064) (layer F.Cu) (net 19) (status C00030))
 (segment (start 145.35 91.65) (end 145 92) (width 0.4064) (layer F.Cu) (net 19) (status C00030))
 (segment (start 145 92) (end 145 91.0625) (width 0.4064) (layer B.Cu) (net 19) (status C00030))
 (segment (start 145 91.0625) (end 145.0625 91) (width 0.4064) (layer B.Cu) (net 19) (status C00030))
 (segment (start 149.0375 92.5) (end 145.5 92.5) (width 0.4064) (layer B.Cu) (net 19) (status C00030))
 (segment (start 145.5 92.5) (end 145 92) (width 0.4064) (layer B.Cu) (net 19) (status C00030))
 (segment (start 130 85) (end 131 85) (width 0.3048) (layer F.Cu) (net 1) (status C00030))
 (segment (start 131.5 85.5) (end 132.55 85.5) (width 0.3048) (layer F.Cu) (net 1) (status 800020))
 (segment (start 131 85) (end 131.5 85.5) (width 0.3048) (layer F.Cu) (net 1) (status 400010))
 (segment (start 130 89.08) (end 130.92 89.08) (width 0.3048) (layer F.Cu) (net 3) (status C00030))
 (segment (start 132.5 87.5) (end 132.55 87.5) (width 0.3048) (layer F.Cu) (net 3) (status C00030))
 (segment (start 130.92 89.08) (end 132.5 87.5) (width 0.3048) (layer F.Cu) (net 3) (status C00030))
 (segment (start 145.45 86) (end 146 86) (width 0.3048) (layer F.Cu) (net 9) (status 400010))
 (segment (start 147 85) (end 148 85) (width 0.3048) (layer F.Cu) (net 9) (status 800030))
 (segment (start 146 86) (end 147 85) (width 0.3048) (layer F.Cu) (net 9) (status 20))
 (segment (start 145.45 88) (end 146.5 88) (width 0.3048) (layer F.Cu) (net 11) (status 400010))
 (segment (start 147.5 89) (end 148 89) (width 0.3048) (layer F.Cu) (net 11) (status C00030))
 (segment (start 146.5 88) (end 147.5 89) (width 0.3048) (layer F.Cu) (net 11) (status 800020))
 (segment (start 141.95 93.6) (end 142.9 93.6) (width 0.2) (layer F.Cu) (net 18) (status 400010))
 (via (at 143.3 95.6) (size 0.6) (drill 0.4) (layers F.Cu B.Cu) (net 18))
 (segment (start 143.3 94.6) (end 143.3 95.6) (width 0.254) (layer F.Cu) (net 18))
 (segment (start 142.9 93.6) (end 143.3 94) (width 0.2) (layer F.Cu) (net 18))
 (segment (start 143.3 94) (end 143.3 94.6) (width 0.2) (layer F.Cu) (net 18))
 (segment (start 142.4 96.5) (end 143.3 95.6) (width 0.254) (layer B.Cu) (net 18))
 (segment (start 139.1 96.5) (end 142.4 96.5) (width 0.254) (layer B.Cu) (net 18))
 (segment (start 136.9 94.3) (end 139.1 96.5) (width 0.254) (layer B.Cu) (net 18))
 (segment (start 135.95 94.05) (end 137 94.05) (width 0.254) (layer F.Cu) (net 18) (status 20))
 (segment (start 135.4 94.1) (end 136.9 94.3) (width 0.254) (layer B.Cu) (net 18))
 (segment (start 135.4 94.1) (end 135.95 94.05) (width 0.254) (layer F.Cu) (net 18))
 (via (at 135.4 94.1) (size 0.6) (drill 0.4) (layers F.Cu B.Cu) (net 18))
 (segment (start 140.9 95.45) (end 140.9 96) (width 0.2) (layer F.Cu) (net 8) (status 400010))
 (segment (start 141.85 96.3) (end 143.55 98) (width 0.254) (layer F.Cu) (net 8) (status 800020))
 (segment (start 141.7 96.3) (end 141.85 96.3) (width 0.254) (layer F.Cu) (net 8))
 (segment (start 140.9 96) (end 141.2 96.3) (width 0.2) (layer F.Cu) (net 8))
 (segment (start 141.2 96.3) (end 141.7 96.3) (width 0.2) (layer F.Cu) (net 8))
 (segment (start 143.5 86.7) (end 143.5 86.05) (width 0.3048) (layer F.Cu) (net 10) (status C00030))
 (segment (start 143.5 86.05) (end 143.55 86) (width 0.3048) (layer F.Cu) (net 10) (status C00030))
 (segment (start 140.9 92.55) (end 140.9 91.5) (width 0.2) (layer F.Cu) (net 10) (status 400010))
 (segment (start 142.7 86.85) (end 143.55 86) (width 0.254) (layer F.Cu) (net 10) (status 800020))
 (segment (start 142.7 90.4) (end 142.7 86.85) (width 0.254) (layer F.Cu) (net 10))
 (segment (start 142.2 90.9) (end 142.7 90.4) (width 0.254) (layer F.Cu) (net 10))
 (segment (start 141.5 90.9) (end 142.2 90.9) (width 0.254) (layer F.Cu) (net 10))
 (segment (start 141.2 91.2) (end 141.5 90.9) (width 0.254) (layer F.Cu) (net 10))
 (segment (start 140.9 91.5) (end 141.2 91.2) (width 0.2) (layer F.Cu) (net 10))
 (segment (start 134.05 100) (end 134.1 100) (width 0.254) (layer F.Cu) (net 16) (status 30))
 (segment (start 134.1 100) (end 134.7 99.4) (width 0.254) (layer F.Cu) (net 16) (status 10))
 (segment (start 134.7 99.4) (end 134.7 97.7) (width 0.254) (layer F.Cu) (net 16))
 (segment (start 134.7 97.7) (end 135.5 96.9) (width 0.254) (layer F.Cu) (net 16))
 (segment (start 135.5 96.9) (end 135.7 96.7) (width 0.254) (layer F.Cu) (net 16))
 (segment (start 135.7 96.7) (end 139.2 96.7) (width 0.254) (layer F.Cu) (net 16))
 (segment (start 140.1 95.45) (end 140.1 96.1) (width 0.2) (layer F.Cu) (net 16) (status 10))
 (segment (start 139.5 96.7) (end 139.2 96.7) (width 0.2) (layer F.Cu) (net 16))
 (segment (start 140.1 96.1) (end 139.5 96.7) (width 0.2) (layer F.Cu) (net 16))
 (segment (start 140.5 95.45) (end 140.5 96.5) (width 0.2) (layer F.Cu) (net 6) (status 400010))
 (segment (start 143 100) (end 143.55 100) (width 0.254) (layer F.Cu) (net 6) (status 800020))
 (segment (start 142.3 99.3) (end 143 100) (width 0.254) (layer F.Cu) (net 6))
 (segment (start 142.3 97.7) (end 142.3 99.3) (width 0.254) (layer F.Cu) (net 6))
 (segment (start 141.4 96.8) (end 142.3 97.7) (width 0.254) (layer F.Cu) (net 6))
 (segment (start 140.8 96.8) (end 141.4 96.8) (width 0.254) (layer F.Cu) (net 6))
 (segment (start 140.5 96.5) (end 140.8 96.8) (width 0.254) (layer F.Cu) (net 6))
 (segment (start 143.5 87.3) (end 143.5 87.95) (width 0.3048) (layer F.Cu) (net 12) (status C00030))
 (segment (start 143.5 87.95) (end 143.55 88) (width 0.3048) (layer F.Cu) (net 12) (status C00030))
 (segment (start 141.3 92.55) (end 141.3 91.8) (width 0.2) (layer F.Cu) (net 12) (status 400010))
 (segment (start 143.4 88.15) (end 143.55 88) (width 0.254) (layer F.Cu) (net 12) (status C00030))
 (segment (start 143.4 90.5) (end 143.4 88.15) (width 0.254) (layer F.Cu) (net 12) (status 800020))
 (segment (start 142.3 91.6) (end 143.4 90.5) (width 0.254) (layer F.Cu) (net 12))
 (segment (start 141.7 91.6) (end 142.3 91.6) (width 0.254) (layer F.Cu) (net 12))
 (segment (start 141.3 91.8) (end 141.5 91.6) (width 0.2) (layer F.Cu) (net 12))
 (segment (start 141.5 91.6) (end 141.7 91.6) (width 0.2) (layer F.Cu) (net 12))
 (segment (start 139.7 92.55) (end 139.15 92.55) (width 0.2) (layer F.Cu) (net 23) (status 400010))
 (segment (start 137 86) (end 137.65 86) (width 0.254) (layer F.Cu) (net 23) (status C00030))
 (segment (start 136.2 86.8) (end 137 86) (width 0.254) (layer F.Cu) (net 23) (status 800020))
 (segment (start 136.2 90.3) (end 136.2 86.8) (width 0.254) (layer F.Cu) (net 23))
 (segment (start 138.8 92.2) (end 138.1 92.2) (width 0.254) (layer F.Cu) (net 23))
 (segment (start 139.15 92.55) (end 138.8 92.2) (width 0.2) (layer F.Cu) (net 23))
 (segment (start 138.1 92.2) (end 136.2 90.3) (width 0.254) (layer F.Cu) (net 23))
 (segment (start 137 95.95) (end 134.45 95.95) (width 0.254) (layer F.Cu) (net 17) (status 400010))
 (segment (start 137.3 96.3) (end 139 98) (width 0.254) (layer B.Cu) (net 17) (status 800020))
 (segment (start 134.3 96.3) (end 137.3 96.3) (width 0.254) (layer B.Cu) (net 17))
 (segment (start 134.2 96.2) (end 134.3 96.3) (width 0.254) (layer B.Cu) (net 17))
 (via (at 134.2 96.2) (size 0.6) (drill 0.4) (layers F.Cu B.Cu) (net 17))
 (segment (start 134.45 95.95) (end 134.2 96.2) (width 0.254) (layer F.Cu) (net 17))
 (segment (start 141.5 88.05) (end 141.5 87.15) (width 0.254) (layer F.Cu) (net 14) (status 400010))
 (segment (start 141.5 87.15) (end 140.35 86) (width 0.254) (layer F.Cu) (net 14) (status 800020))
 (segment (start 135.95 100) (end 137.65 100) (width 0.3048) (layer F.Cu) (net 15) (status C00030))
 (segment (start 134.45 86.85) (end 134.5 86.8) (width 0.3048) (layer F.Cu) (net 4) (status C00030))
 (segment (start 134.45 87.5) (end 134.45 86.85) (width 0.3048) (layer F.Cu) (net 4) (status C00030))
 (segment (start 134.45 87.5) (end 134.45 88.85) (width 0.254) (layer F.Cu) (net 4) (status 10))
 (segment (start 134.45 88.85) (end 133.3 90) (width 0.254) (layer F.Cu) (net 4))
 (segment (start 133.3 90) (end 133.3 93.7) (width 0.254) (layer F.Cu) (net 4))
 (segment (start 134.4 94.8) (end 134.9 94.8) (width 0.254) (layer F.Cu) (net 4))
 (segment (start 134.9 94.8) (end 134.918989 94.818989) (width 0.254) (layer F.Cu) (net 4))
 (segment (start 133.3 93.7) (end 134.4 94.8) (width 0.254) (layer F.Cu) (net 4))
 (segment (start 134.9 94.8) (end 137.6 94.8) (width 0.254) (layer F.Cu) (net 4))
 (segment (start 139.05 94.4) (end 138.1 94.4) (width 0.2) (layer F.Cu) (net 4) (status 10))
 (segment (start 137.7 94.8) (end 137.6 94.8) (width 0.2) (layer F.Cu) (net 4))
 (segment (start 138.1 94.4) (end 137.7 94.8) (width 0.2) (layer F.Cu) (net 4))
 (segment (start 132.9 98.3) (end 133.74599 98.3) (width 0.254) (layer F.Cu) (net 24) (status 30))
 (segment (start 133.9 98.3) (end 133.9 97.3) (width 0.254) (layer F.Cu) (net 24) (status 10))
 (segment (start 133.572999 95.899039) (end 134.199039 95.272999) (width 0.254) (layer F.Cu) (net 24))
 (segment (start 133.572999 96.972999) (end 133.572999 95.899039) (width 0.254) (layer F.Cu) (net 24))
 (segment (start 133.9 97.3) (end 133.572999 96.972999) (width 0.254) (layer F.Cu) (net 24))
 (segment (start 134.199039 95.272999) (end 136.088399 95.272999) (width 0.254) (layer F.Cu) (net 24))
 (segment (start 136.088399 95.272999) (end 137.7 95.272999) (width 0.254) (layer F.Cu) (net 24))
 (segment (start 137.827001 95.272999) (end 137.7 95.272999) (width 0.2) (layer F.Cu) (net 24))
 (segment (start 138.3 94.8) (end 137.827001 95.272999) (width 0.2) (layer F.Cu) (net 24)))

